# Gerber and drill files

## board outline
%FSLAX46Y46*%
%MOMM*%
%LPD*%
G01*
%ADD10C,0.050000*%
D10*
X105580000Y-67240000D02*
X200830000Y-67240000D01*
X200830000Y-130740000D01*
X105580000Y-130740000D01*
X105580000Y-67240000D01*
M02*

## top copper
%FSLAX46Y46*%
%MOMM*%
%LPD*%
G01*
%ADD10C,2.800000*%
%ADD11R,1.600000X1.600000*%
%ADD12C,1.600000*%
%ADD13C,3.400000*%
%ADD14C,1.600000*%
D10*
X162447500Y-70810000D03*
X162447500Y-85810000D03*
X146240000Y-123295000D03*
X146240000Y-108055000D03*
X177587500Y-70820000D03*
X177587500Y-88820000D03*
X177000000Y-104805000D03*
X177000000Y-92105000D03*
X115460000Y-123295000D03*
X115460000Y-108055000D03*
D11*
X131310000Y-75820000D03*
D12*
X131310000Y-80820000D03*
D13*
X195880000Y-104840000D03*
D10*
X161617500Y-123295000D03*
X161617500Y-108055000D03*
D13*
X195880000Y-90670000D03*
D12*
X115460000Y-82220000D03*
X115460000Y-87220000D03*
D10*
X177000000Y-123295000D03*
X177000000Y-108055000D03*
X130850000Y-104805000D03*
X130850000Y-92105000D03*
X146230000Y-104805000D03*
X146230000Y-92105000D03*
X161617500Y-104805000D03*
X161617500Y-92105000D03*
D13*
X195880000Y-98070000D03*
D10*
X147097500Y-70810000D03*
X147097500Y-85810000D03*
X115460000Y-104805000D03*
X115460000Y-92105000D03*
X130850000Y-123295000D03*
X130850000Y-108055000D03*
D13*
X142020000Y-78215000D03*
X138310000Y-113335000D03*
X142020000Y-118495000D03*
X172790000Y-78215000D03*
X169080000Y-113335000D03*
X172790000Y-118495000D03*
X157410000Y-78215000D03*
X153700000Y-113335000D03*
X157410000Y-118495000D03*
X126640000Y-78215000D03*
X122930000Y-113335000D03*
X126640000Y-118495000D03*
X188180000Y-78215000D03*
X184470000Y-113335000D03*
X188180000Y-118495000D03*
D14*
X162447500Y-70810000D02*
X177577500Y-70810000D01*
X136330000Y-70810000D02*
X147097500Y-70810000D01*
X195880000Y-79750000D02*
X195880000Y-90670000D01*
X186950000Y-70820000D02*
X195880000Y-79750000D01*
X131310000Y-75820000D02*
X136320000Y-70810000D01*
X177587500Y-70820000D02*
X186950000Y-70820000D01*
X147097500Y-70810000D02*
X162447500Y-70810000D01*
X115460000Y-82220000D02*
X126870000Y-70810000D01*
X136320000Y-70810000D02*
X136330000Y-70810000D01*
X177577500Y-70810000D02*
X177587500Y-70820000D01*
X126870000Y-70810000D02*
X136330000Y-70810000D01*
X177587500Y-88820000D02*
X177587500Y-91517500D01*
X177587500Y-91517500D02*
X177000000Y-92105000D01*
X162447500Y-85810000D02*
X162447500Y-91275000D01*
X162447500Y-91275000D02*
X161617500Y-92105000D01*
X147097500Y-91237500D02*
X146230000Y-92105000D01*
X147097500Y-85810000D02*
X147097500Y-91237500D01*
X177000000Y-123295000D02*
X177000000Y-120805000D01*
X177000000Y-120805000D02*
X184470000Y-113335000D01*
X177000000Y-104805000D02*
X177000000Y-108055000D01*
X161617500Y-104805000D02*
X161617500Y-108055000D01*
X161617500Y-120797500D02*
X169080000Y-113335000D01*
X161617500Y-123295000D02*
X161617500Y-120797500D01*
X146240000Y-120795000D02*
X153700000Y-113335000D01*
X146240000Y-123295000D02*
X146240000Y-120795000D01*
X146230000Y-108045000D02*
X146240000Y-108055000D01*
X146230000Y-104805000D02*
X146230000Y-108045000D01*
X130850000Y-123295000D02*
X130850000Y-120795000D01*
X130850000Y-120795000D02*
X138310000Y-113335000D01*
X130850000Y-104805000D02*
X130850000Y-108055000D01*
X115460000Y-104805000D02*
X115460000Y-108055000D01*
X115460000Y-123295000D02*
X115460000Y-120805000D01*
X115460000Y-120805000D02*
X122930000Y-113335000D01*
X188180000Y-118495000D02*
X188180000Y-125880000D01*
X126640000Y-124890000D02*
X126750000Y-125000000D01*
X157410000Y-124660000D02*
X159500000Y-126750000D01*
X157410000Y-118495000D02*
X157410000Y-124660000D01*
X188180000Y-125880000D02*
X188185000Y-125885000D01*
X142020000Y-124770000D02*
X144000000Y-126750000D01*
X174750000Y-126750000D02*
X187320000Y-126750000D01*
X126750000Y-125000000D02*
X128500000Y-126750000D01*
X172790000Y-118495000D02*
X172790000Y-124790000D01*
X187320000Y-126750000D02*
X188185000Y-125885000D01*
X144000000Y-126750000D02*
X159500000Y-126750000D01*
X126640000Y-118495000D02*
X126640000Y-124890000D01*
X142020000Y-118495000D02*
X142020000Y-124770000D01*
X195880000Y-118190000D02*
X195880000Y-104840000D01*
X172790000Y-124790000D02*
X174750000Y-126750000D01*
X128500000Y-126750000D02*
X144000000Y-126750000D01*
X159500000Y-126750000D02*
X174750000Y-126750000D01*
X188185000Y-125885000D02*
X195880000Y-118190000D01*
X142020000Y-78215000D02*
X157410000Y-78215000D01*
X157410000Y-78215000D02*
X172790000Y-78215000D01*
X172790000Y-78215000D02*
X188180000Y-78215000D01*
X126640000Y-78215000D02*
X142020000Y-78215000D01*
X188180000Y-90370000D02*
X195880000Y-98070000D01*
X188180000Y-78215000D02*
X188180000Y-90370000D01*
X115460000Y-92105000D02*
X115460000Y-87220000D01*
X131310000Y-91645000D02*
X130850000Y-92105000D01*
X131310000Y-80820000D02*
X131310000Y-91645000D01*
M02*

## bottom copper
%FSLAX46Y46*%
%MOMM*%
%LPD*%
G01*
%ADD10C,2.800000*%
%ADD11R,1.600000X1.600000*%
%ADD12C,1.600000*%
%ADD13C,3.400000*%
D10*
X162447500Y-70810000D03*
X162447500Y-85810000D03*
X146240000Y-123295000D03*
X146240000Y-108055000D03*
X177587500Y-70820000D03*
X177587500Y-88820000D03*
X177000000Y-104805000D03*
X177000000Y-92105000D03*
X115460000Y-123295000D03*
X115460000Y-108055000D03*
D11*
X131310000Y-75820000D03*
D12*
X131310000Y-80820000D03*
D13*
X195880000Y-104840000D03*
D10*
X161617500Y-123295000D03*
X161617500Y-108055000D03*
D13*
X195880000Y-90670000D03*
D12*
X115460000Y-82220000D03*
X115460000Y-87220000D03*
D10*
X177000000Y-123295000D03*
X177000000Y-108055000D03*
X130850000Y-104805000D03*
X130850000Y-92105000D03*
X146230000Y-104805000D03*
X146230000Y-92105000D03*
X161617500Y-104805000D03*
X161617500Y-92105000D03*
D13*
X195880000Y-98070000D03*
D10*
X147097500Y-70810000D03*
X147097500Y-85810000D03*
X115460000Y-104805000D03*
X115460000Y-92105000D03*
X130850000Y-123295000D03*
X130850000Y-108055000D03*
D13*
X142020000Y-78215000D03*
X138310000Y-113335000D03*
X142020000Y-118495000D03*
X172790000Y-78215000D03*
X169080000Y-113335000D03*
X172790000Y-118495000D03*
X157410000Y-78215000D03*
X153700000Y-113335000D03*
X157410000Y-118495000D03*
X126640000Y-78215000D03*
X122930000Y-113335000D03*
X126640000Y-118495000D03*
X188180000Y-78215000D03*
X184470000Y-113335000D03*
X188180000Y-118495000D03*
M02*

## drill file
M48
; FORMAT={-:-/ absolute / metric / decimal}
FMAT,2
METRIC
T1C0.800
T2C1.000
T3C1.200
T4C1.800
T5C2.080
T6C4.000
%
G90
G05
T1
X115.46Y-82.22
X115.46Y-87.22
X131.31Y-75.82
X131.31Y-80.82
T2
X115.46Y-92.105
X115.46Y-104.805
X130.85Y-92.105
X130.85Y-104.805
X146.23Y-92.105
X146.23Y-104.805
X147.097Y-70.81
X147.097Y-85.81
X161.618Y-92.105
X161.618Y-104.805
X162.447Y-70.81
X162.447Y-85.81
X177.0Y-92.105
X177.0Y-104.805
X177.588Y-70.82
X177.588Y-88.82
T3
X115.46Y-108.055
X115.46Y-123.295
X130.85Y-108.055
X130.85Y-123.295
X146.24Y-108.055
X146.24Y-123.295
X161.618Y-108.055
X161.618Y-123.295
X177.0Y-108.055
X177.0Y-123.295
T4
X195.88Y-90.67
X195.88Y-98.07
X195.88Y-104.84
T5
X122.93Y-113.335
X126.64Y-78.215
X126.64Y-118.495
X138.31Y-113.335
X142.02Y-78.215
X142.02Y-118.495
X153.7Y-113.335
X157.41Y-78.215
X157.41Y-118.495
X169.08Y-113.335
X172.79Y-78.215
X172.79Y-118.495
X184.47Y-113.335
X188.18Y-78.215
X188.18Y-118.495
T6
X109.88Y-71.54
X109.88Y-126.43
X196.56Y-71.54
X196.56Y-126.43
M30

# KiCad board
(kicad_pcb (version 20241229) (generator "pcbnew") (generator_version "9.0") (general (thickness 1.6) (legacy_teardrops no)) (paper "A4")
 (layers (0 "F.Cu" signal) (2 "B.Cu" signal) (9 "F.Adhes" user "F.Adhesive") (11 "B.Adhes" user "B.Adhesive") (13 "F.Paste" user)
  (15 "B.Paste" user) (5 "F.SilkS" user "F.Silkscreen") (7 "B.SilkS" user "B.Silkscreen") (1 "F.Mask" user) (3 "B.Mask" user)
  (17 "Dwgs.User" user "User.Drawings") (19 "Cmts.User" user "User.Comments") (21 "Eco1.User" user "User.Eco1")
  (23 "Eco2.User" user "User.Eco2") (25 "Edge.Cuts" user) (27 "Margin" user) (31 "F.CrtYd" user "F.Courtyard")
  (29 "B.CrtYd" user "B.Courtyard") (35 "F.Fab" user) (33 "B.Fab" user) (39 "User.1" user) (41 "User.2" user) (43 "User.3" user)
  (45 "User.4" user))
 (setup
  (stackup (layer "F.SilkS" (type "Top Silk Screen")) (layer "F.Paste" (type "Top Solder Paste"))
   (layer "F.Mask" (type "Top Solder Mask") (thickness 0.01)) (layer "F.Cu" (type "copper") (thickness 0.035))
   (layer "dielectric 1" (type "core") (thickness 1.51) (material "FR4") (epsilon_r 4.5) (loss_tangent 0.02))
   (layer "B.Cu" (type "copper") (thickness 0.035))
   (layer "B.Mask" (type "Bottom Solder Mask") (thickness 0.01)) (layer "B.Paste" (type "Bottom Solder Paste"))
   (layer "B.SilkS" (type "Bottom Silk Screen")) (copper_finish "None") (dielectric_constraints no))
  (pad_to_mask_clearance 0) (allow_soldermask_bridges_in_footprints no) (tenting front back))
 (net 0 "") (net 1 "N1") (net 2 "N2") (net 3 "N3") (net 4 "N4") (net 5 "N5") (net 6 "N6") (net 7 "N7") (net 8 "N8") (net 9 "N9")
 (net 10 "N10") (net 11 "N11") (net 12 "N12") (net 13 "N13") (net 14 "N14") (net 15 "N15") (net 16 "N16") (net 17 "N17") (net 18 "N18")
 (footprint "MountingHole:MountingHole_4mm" (layer "F.Cu") (at 196.56 126.43)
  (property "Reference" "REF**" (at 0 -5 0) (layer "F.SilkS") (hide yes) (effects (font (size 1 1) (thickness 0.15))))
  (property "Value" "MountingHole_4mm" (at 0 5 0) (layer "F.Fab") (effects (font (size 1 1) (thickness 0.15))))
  (pad "" np_thru_hole circle (at 0 0) (size 4 4) (drill 4) (layers "*.Cu" "*.Mask")))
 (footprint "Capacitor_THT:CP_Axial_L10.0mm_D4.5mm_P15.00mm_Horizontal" (layer "F.Cu") (at 162.4475 70.81 -90)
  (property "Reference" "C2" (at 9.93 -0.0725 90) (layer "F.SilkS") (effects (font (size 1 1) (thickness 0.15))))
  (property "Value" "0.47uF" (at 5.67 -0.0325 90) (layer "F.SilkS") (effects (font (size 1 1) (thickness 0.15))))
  (pad "1" thru_hole circle (at 0 0 270) (size 2.8 2.8) (drill 1) (layers "*.Cu" "*.Mask") (remove_unused_layers no) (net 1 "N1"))
  (pad "2" thru_hole circle (at 15 0 270) (size 2.8 2.8) (drill 1) (layers "*.Cu" "*.Mask") (remove_unused_layers no) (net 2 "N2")))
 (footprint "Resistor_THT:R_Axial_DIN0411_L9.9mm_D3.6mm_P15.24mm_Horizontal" (layer "F.Cu") (at 146.24 123.295 90)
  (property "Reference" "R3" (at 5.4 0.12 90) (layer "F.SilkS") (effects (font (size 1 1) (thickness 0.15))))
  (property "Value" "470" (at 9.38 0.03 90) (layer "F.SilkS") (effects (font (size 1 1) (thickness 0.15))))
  (pad "1" thru_hole circle (at 0 0 90) (size 2.8 2.8) (drill 1.2) (layers "*.Cu" "*.Mask") (remove_unused_layers no) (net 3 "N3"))
  (pad "2" thru_hole circle (at 15.24 0 90) (size 2.8 2.8) (drill 1.2) (layers "*.Cu" "*.Mask") (remove_unused_layers no) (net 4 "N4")))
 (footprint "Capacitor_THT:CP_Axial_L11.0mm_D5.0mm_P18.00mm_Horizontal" (layer "F.Cu") (at 177.5875 70.82 -90)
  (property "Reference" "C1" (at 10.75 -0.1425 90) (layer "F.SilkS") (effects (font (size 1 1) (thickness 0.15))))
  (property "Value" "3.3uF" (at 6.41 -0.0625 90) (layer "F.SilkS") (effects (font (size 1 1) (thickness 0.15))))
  (pad "1" thru_hole circle (at 0 0 270) (size 2.8 2.8) (drill 1) (layers "*.Cu" "*.Mask") (remove_unused_layers no) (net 1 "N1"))
  (pad "2" thru_hole circle (at 18 0 270) (size 2.8 2.8) (drill 1) (layers "*.Cu" "*.Mask") (remove_unused_layers no) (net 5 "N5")))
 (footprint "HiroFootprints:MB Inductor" (layer "F.Cu") (at 177 104.805 90)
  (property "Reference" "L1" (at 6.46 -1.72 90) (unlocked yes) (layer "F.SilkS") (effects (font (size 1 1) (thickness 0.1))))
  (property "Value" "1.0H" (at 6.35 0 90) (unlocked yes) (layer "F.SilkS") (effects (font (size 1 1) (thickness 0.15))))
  (pad "1" thru_hole circle (at 0 0 90) (size 2.8 2.8) (drill 1) (layers "*.Cu" "*.Mask") (remove_unused_layers no) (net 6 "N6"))
  (pad "2" thru_hole circle (at 12.7 0 90) (size 2.8 2.8) (drill 1) (layers "*.Cu" "*.Mask") (remove_unused_layers no) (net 5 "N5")))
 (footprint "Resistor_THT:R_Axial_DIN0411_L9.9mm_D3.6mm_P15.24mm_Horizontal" (layer "F.Cu") (at 115.46 123.295 90)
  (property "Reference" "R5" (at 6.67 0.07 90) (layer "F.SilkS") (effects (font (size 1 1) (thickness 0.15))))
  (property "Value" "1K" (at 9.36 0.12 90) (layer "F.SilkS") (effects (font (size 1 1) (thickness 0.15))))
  (pad "1" thru_hole circle (at 0 0 90) (size 2.8 2.8) (drill 1.2) (layers "*.Cu" "*.Mask") (remove_unused_layers no) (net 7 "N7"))
  (pad "2" thru_hole circle (at 15.24 0 90) (size 2.8 2.8) (drill 1.2) (layers "*.Cu" "*.Mask") (remove_unused_layers no) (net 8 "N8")))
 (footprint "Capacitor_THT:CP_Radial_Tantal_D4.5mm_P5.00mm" (layer "F.Cu") (at 131.31 75.82 -90)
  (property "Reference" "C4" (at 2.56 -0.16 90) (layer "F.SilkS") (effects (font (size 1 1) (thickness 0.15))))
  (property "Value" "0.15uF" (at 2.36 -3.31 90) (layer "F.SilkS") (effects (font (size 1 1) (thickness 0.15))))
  (pad "1" thru_hole rect (at 0 0 270) (size 1.6 1.6) (drill 0.8) (layers "*.Cu" "*.Mask") (remove_unused_layers no) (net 1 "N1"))
  (pad "2" thru_hole circle (at 5 0 270) (size 1.6 1.6) (drill 0.8) (layers "*.Cu" "*.Mask") (remove_unused_layers no) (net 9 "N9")))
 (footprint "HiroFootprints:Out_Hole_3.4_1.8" (layer "F.Cu") (at 195.88 104.84)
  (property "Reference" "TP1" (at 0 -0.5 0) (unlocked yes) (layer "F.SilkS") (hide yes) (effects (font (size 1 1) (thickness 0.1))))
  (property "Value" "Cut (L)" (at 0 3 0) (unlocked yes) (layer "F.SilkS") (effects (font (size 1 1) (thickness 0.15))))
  (pad "1" thru_hole circle (at 0 0) (size 3.4 3.4) (drill 1.8) (layers "*.Cu" "*.Mask") (remove_unused_layers no) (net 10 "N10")))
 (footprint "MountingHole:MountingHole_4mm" (layer "F.Cu") (at 109.88 71.54)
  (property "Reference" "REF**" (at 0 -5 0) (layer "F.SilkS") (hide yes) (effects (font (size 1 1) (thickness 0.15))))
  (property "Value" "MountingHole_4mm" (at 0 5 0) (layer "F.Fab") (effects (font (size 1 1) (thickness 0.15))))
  (pad "" np_thru_hole circle (at 0 0) (size 4 4) (drill 4) (layers "*.Cu" "*.Mask")))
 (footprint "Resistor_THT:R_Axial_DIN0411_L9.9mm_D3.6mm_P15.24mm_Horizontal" (layer "F.Cu") (at 161.6175 123.295 90)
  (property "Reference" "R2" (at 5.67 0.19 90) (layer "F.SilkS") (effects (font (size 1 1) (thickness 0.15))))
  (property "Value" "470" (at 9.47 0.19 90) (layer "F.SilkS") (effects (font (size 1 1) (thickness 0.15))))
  (pad "1" thru_hole circle (at 0 0 90) (size 2.8 2.8) (drill 1.2) (layers "*.Cu" "*.Mask") (remove_unused_layers no) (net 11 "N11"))
  (pad "2" thru_hole circle (at 15.24 0 90) (size 2.8 2.8) (drill 1.2) (layers "*.Cu" "*.Mask") (remove_unused_layers no) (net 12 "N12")))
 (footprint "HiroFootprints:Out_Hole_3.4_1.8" (layer "F.Cu") (at 195.88 90.67)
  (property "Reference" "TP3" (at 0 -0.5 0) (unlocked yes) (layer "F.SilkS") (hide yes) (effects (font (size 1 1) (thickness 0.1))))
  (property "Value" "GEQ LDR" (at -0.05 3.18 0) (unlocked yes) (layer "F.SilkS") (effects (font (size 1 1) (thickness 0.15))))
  (pad "1" thru_hole circle (at 0 0) (size 3.4 3.4) (drill 1.8) (layers "*.Cu" "*.Mask") (remove_unused_layers no) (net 1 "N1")))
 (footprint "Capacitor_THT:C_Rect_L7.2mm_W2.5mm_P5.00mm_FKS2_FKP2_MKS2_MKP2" (layer "F.Cu") (at 115.46 82.22 -90)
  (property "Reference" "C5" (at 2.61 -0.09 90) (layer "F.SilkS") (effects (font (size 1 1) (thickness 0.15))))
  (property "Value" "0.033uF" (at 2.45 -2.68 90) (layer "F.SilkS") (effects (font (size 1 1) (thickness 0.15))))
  (pad "1" thru_hole circle (at 0 0 270) (size 1.6 1.6) (drill 0.8) (layers "*.Cu" "*.Mask") (remove_unused_layers no) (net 1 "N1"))
  (pad "2" thru_hole circle (at 5 0 270) (size 1.6 1.6) (drill 0.8) (layers "*.Cu" "*.Mask") (remove_unused_layers no) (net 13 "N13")))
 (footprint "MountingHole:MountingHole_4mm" (layer "F.Cu") (at 196.56 71.54)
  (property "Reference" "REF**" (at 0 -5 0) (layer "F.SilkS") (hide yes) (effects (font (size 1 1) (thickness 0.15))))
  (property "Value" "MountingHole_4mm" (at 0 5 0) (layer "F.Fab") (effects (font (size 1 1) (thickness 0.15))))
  (pad "" np_thru_hole circle (at 0 0) (size 4 4) (drill 4) (layers "*.Cu" "*.Mask")))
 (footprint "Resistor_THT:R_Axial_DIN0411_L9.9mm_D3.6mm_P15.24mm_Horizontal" (layer "F.Cu") (at 177 123.295 90)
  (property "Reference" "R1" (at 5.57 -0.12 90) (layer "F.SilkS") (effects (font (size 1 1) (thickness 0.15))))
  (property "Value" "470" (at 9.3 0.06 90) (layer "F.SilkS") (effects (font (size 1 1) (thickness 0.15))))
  (pad "1" thru_hole circle (at 0 0 90) (size 2.8 2.8) (drill 1.2) (layers "*.Cu" "*.Mask") (remove_unused_layers no) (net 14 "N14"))
  (pad "2" thru_hole circle (at 15.24 0 90) (size 2.8 2.8) (drill 1.2) (layers "*.Cu" "*.Mask") (remove_unused_layers no) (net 6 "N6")))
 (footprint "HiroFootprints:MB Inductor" (layer "F.Cu") (at 130.85 104.805 90)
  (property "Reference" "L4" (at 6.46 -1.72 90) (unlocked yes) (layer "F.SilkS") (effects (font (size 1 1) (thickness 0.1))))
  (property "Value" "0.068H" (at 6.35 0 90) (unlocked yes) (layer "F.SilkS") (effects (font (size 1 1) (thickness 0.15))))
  (pad "1" thru_hole circle (at 0 0 90) (size 2.8 2.8) (drill 1) (layers "*.Cu" "*.Mask") (remove_unused_layers no) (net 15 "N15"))
  (pad "2" thru_hole circle (at 12.7 0 90) (size 2.8 2.8) (drill 1) (layers "*.Cu" "*.Mask") (remove_unused_layers no) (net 9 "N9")))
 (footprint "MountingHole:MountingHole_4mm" (layer "F.Cu") (at 109.88 126.43)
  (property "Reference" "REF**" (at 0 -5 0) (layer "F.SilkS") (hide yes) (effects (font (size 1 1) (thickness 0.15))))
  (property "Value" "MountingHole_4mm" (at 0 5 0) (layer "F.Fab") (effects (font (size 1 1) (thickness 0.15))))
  (pad "" np_thru_hole circle (at 0 0) (size 4 4) (drill 4) (layers "*.Cu" "*.Mask")))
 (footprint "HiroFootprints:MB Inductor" (layer "F.Cu") (at 146.23 104.805 90)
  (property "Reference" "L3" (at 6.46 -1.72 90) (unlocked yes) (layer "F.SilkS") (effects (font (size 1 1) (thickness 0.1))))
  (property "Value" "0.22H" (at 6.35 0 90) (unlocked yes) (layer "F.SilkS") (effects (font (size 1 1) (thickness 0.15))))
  (pad "1" thru_hole circle (at 0 0 90) (size 2.8 2.8) (drill 1) (layers "*.Cu" "*.Mask") (remove_unused_layers no) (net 4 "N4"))
  (pad "2" thru_hole circle (at 12.7 0 90) (size 2.8 2.8) (drill 1) (layers "*.Cu" "*.Mask") (remove_unused_layers no) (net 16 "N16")))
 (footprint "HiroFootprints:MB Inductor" (layer "F.Cu") (at 161.6175 104.805 90)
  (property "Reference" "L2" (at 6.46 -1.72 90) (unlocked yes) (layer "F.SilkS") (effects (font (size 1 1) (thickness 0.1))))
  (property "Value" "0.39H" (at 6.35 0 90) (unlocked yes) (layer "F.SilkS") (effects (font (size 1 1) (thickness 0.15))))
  (pad "1" thru_hole circle (at 0 0 90) (size 2.8 2.8) (drill 1) (layers "*.Cu" "*.Mask") (remove_unused_layers no) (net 12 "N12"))
  (pad "2" thru_hole circle (at 12.7 0 90) (size 2.8 2.8) (drill 1) (layers "*.Cu" "*.Mask") (remove_unused_layers no) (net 2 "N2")))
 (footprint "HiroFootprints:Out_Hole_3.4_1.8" (layer "F.Cu") (at 195.88 98.07)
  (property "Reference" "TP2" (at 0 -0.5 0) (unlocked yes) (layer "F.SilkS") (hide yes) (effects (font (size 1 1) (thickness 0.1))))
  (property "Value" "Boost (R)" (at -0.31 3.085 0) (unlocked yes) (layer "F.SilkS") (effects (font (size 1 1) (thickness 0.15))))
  (pad "1" thru_hole circle (at 0 0) (size 3.4 3.4) (drill 1.8) (layers "*.Cu" "*.Mask") (remove_unused_layers no) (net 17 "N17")))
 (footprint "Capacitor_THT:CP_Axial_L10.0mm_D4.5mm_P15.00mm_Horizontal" (layer "F.Cu") (at 147.0975 70.81 -90)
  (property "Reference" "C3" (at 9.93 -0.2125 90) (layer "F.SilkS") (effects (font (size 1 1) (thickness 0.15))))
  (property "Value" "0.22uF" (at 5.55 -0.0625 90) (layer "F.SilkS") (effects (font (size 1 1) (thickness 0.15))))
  (pad "1" thru_hole circle (at 0 0 270) (size 2.8 2.8) (drill 1) (layers "*.Cu" "*.Mask") (remove_unused_layers no) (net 1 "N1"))
  (pad "2" thru_hole circle (at 15 0 270) (size 2.8 2.8) (drill 1) (layers "*.Cu" "*.Mask") (remove_unused_layers no) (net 16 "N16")))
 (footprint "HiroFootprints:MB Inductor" (layer "F.Cu") (at 115.46 104.805 90)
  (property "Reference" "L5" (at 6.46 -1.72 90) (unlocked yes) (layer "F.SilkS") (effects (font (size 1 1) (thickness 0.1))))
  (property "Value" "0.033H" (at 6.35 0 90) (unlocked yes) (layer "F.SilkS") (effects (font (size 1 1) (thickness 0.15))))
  (pad "1" thru_hole circle (at 0 0 90) (size 2.8 2.8) (drill 1) (layers "*.Cu" "*.Mask") (remove_unused_layers no) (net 8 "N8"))
  (pad "2" thru_hole circle (at 12.7 0 90) (size 2.8 2.8) (drill 1) (layers "*.Cu" "*.Mask") (remove_unused_layers no) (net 13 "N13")))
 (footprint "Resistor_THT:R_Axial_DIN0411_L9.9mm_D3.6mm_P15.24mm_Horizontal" (layer "F.Cu") (at 130.85 123.295 90)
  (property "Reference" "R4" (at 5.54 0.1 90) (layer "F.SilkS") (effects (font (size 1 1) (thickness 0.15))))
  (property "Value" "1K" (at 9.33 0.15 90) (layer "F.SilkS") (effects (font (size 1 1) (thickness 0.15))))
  (pad "1" thru_hole circle (at 0 0 90) (size 2.8 2.8) (drill 1.2) (layers "*.Cu" "*.Mask") (remove_unused_layers no) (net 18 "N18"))
  (pad "2" thru_hole circle (at 15.24 0 90) (size 2.8 2.8) (drill 1.2) (layers "*.Cu" "*.Mask") (remove_unused_layers no) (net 15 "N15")))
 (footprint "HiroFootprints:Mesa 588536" (layer "B.Cu") (at 142.02 124.035 -90)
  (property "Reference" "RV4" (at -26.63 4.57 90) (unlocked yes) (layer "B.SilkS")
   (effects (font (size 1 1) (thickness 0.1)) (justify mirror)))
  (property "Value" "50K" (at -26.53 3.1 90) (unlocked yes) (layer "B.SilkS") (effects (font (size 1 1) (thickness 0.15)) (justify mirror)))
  (pad "1" thru_hole circle (at -45.82 0 270) (size 3.4 3.4) (drill 2.08) (layers "*.Cu" "*.Mask") (remove_unused_layers no) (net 17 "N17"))
  (pad "2" thru_hole circle (at -10.7 3.71 270) (size 3.4 3.4) (drill 2.08) (layers "*.Cu" "*.Mask") (remove_unused_layers no)
   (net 18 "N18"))
  (pad "3" thru_hole circle (at -5.54 0 270) (size 3.4 3.4) (drill 2.08) (layers "*.Cu" "*.Mask") (remove_unused_layers no) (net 10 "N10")))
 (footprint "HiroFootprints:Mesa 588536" (layer "B.Cu") (at 172.79 124.035 -90)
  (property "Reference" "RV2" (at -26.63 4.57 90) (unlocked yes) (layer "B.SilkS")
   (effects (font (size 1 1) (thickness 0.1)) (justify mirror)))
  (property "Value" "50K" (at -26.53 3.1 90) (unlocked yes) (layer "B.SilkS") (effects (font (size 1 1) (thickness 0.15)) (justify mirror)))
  (pad "1" thru_hole circle (at -45.82 0 270) (size 3.4 3.4) (drill 2.08) (layers "*.Cu" "*.Mask") (remove_unused_layers no) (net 17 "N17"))
  (pad "2" thru_hole circle (at -10.7 3.71 270) (size 3.4 3.4) (drill 2.08) (layers "*.Cu" "*.Mask") (remove_unused_layers no)
   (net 11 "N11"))
  (pad "3" thru_hole circle (at -5.54 0 270) (size 3.4 3.4) (drill 2.08) (layers "*.Cu" "*.Mask") (remove_unused_layers no) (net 10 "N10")))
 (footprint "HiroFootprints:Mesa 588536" (layer "B.Cu") (at 157.41 124.035 -90)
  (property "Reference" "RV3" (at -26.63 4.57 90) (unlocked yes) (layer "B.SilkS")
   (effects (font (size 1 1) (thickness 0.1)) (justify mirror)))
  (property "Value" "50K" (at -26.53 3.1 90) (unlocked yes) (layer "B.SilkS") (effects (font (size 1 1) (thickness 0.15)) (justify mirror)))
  (pad "1" thru_hole circle (at -45.82 0 270) (size 3.4 3.4) (drill 2.08) (layers "*.Cu" "*.Mask") (remove_unused_layers no) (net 17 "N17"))
  (pad "2" thru_hole circle (at -10.7 3.71 270) (size 3.4 3.4) (drill 2.08) (layers "*.Cu" "*.Mask") (remove_unused_layers no) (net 3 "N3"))
  (pad "3" thru_hole circle (at -5.54 0 270) (size 3.4 3.4) (drill 2.08) (layers "*.Cu" "*.Mask") (remove_unused_layers no) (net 10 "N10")))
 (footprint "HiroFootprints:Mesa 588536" (layer "B.Cu") (at 126.64 124.035 -90)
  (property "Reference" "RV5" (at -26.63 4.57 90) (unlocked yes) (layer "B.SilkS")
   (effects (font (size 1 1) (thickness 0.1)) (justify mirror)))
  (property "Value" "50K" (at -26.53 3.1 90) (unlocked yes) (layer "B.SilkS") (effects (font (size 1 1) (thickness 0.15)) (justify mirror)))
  (pad "1" thru_hole circle (at -45.82 0 270) (size 3.4 3.4) (drill 2.08) (layers "*.Cu" "*.Mask") (remove_unused_layers no) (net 17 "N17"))
  (pad "2" thru_hole circle (at -10.7 3.71 270) (size 3.4 3.4) (drill 2.08) (layers "*.Cu" "*.Mask") (remove_unused_layers no) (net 7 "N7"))
  (pad "3" thru_hole circle (at -5.54 0 270) (size 3.4 3.4) (drill 2.08) (layers "*.Cu" "*.Mask") (remove_unused_layers no) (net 10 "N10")))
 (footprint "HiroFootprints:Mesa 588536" (layer "B.Cu") (at 188.18 124.035 -90)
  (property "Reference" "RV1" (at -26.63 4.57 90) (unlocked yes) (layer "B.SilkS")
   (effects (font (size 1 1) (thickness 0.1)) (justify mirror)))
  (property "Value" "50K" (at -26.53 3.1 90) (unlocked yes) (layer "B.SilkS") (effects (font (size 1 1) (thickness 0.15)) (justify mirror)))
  (pad "1" thru_hole circle (at -45.82 0 270) (size 3.4 3.4) (drill 2.08) (layers "*.Cu" "*.Mask") (remove_unused_layers no) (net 17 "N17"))
  (pad "2" thru_hole circle (at -10.7 3.71 270) (size 3.4 3.4) (drill 2.08) (layers "*.Cu" "*.Mask") (remove_unused_layers no)
   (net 14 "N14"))
  (pad "3" thru_hole circle (at -5.54 0 270) (size 3.4 3.4) (drill 2.08) (layers "*.Cu" "*.Mask") (remove_unused_layers no) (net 10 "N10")))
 (gr_rect (start 105.58 67.24) (end 200.83 130.74) (stroke (width 0.05) (type solid)) (fill no) (layer "Edge.Cuts"))
 (segment (start 162.4475 70.81) (end 177.5775 70.81) (width 1.6) (layer "F.Cu") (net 1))
 (segment (start 136.33 70.81) (end 147.0975 70.81) (width 1.6) (layer "F.Cu") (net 1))
 (segment (start 195.88 79.75) (end 195.88 90.67) (width 1.6) (layer "F.Cu") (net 1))
 (segment (start 186.95 70.82) (end 195.88 79.75) (width 1.6) (layer "F.Cu") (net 1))
 (segment (start 131.31 75.82) (end 136.32 70.81) (width 1.6) (layer "F.Cu") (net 1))
 (segment (start 177.5875 70.82) (end 186.95 70.82) (width 1.6) (layer "F.Cu") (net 1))
 (segment (start 147.0975 70.81) (end 162.4475 70.81) (width 1.6) (layer "F.Cu") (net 1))
 (segment (start 115.46 82.22) (end 126.87 70.81) (width 1.6) (layer "F.Cu") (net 1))
 (segment (start 136.32 70.81) (end 136.33 70.81) (width 1.6) (layer "F.Cu") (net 1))
 (segment (start 177.5775 70.81) (end 177.5875 70.82) (width 1.6) (layer "F.Cu") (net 1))
 (segment (start 126.87 70.81) (end 136.33 70.81) (width 1.6) (layer "F.Cu") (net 1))
 (segment (start 177.5875 88.82) (end 177.5875 91.5175) (width 1.6) (layer "F.Cu") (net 5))
 (segment (start 177.5875 91.5175) (end 177 92.105) (width 1.6) (layer "F.Cu") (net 5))
 (segment (start 162.4475 85.81) (end 162.4475 91.275) (width 1.6) (layer "F.Cu") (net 2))
 (segment (start 162.4475 91.275) (end 161.6175 92.105) (width 1.6) (layer "F.Cu") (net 2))
 (segment (start 147.0975 91.2375) (end 146.23 92.105) (width 1.6) (layer "F.Cu") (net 16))
 (segment (start 147.0975 85.81) (end 147.0975 91.2375) (width 1.6) (layer "F.Cu") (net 16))
 (segment (start 177 123.295) (end 177 120.805) (width 1.6) (layer "F.Cu") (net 14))
 (segment (start 177 120.805) (end 184.47 113.335) (width 1.6) (layer "F.Cu") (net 14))
 (segment (start 177 104.805) (end 177 108.055) (width 1.6) (layer "F.Cu") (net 6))
 (segment (start 161.6175 104.805) (end 161.6175 108.055) (width 1.6) (layer "F.Cu") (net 12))
 (segment (start 161.6175 120.7975) (end 169.08 113.335) (width 1.6) (layer "F.Cu") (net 11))
 (segment (start 161.6175 123.295) (end 161.6175 120.7975) (width 1.6) (layer "F.Cu") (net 11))
 (segment (start 146.24 120.795) (end 153.7 113.335) (width 1.6) (layer "F.Cu") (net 3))
 (segment (start 146.24 123.295) (end 146.24 120.795) (width 1.6) (layer "F.Cu") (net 3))
 (segment (start 146.23 108.045) (end 146.24 108.055) (width 1.6) (layer "F.Cu") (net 4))
 (segment (start 146.23 104.805) (end 146.23 108.045) (width 1.6) (layer "F.Cu") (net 4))
 (segment (start 130.85 123.295) (end 130.85 120.795) (width 1.6) (layer "F.Cu") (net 18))
 (segment (start 130.85 120.795) (end 138.31 113.335) (width 1.6) (layer "F.Cu") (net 18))
 (segment (start 130.85 104.805) (end 130.85 108.055) (width 1.6) (layer "F.Cu") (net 15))
 (segment (start 115.46 104.805) (end 115.46 108.055) (width 1.6) (layer "F.Cu") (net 8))
 (segment (start 115.46 123.295) (end 115.46 120.805) (width 1.6) (layer "F.Cu") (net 7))
 (segment (start 115.46 120.805) (end 122.93 113.335) (width 1.6) (layer "F.Cu") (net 7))
 (segment (start 188.18 118.495) (end 188.18 125.88) (width 1.6) (layer "F.Cu") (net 10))
 (segment (start 126.64 124.89) (end 126.75 125) (width 1.6) (layer "F.Cu") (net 10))
 (segment (start 157.41 124.66) (end 159.5 126.75) (width 1.6) (layer "F.Cu") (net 10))
 (segment (start 157.41 118.495) (end 157.41 124.66) (width 1.6) (layer "F.Cu") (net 10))
 (segment (start 188.18 125.88) (end 188.185 125.885) (width 1.6) (layer "F.Cu") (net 10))
 (segment (start 142.02 124.77) (end 144 126.75) (width 1.6) (layer "F.Cu") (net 10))
 (segment (start 174.75 126.75) (end 187.32 126.75) (width 1.6) (layer "F.Cu") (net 10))
 (segment (start 126.75 125) (end 128.5 126.75) (width 1.6) (layer "F.Cu") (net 10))
 (segment (start 172.79 118.495) (end 172.79 124.79) (width 1.6) (layer "F.Cu") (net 10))
 (segment (start 187.32 126.75) (end 188.185 125.885) (width 1.6) (layer "F.Cu") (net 10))
 (segment (start 144 126.75) (end 159.5 126.75) (width 1.6) (layer "F.Cu") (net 10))
 (segment (start 126.64 118.495) (end 126.64 124.89) (width 1.6) (layer "F.Cu") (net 10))
 (segment (start 142.02 118.495) (end 142.02 124.77) (width 1.6) (layer "F.Cu") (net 10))
 (segment (start 195.88 118.19) (end 195.88 104.84) (width 1.6) (layer "F.Cu") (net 10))
 (segment (start 172.79 124.79) (end 174.75 126.75) (width 1.6) (layer "F.Cu") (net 10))
 (segment (start 128.5 126.75) (end 144 126.75) (width 1.6) (layer "F.Cu") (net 10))
 (segment (start 159.5 126.75) (end 174.75 126.75) (width 1.6) (layer "F.Cu") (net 10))
 (segment (start 188.185 125.885) (end 195.88 118.19) (width 1.6) (layer "F.Cu") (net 10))
 (segment (start 142.02 78.215) (end 157.41 78.215) (width 1.6) (layer "F.Cu") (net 17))
 (segment (start 157.41 78.215) (end 172.79 78.215) (width 1.6) (layer "F.Cu") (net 17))
 (segment (start 172.79 78.215) (end 188.18 78.215) (width 1.6) (layer "F.Cu") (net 17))
 (segment (start 126.64 78.215) (end 142.02 78.215) (width 1.6) (layer "F.Cu") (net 17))
 (segment (start 188.18 90.37) (end 195.88 98.07) (width 1.6) (layer "F.Cu") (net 17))
 (segment (start 188.18 78.215) (end 188.18 90.37) (width 1.6) (layer "F.Cu") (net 17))
 (segment (start 115.46 92.105) (end 115.46 87.22) (width 1.6) (layer "F.Cu") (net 13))
 (segment (start 131.31 91.645) (end 130.85 92.105) (width 1.6) (layer "F.Cu") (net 9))
 (segment (start 131.31 80.82) (end 131.31 91.645) (width 1.6) (layer "F.Cu") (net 9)))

